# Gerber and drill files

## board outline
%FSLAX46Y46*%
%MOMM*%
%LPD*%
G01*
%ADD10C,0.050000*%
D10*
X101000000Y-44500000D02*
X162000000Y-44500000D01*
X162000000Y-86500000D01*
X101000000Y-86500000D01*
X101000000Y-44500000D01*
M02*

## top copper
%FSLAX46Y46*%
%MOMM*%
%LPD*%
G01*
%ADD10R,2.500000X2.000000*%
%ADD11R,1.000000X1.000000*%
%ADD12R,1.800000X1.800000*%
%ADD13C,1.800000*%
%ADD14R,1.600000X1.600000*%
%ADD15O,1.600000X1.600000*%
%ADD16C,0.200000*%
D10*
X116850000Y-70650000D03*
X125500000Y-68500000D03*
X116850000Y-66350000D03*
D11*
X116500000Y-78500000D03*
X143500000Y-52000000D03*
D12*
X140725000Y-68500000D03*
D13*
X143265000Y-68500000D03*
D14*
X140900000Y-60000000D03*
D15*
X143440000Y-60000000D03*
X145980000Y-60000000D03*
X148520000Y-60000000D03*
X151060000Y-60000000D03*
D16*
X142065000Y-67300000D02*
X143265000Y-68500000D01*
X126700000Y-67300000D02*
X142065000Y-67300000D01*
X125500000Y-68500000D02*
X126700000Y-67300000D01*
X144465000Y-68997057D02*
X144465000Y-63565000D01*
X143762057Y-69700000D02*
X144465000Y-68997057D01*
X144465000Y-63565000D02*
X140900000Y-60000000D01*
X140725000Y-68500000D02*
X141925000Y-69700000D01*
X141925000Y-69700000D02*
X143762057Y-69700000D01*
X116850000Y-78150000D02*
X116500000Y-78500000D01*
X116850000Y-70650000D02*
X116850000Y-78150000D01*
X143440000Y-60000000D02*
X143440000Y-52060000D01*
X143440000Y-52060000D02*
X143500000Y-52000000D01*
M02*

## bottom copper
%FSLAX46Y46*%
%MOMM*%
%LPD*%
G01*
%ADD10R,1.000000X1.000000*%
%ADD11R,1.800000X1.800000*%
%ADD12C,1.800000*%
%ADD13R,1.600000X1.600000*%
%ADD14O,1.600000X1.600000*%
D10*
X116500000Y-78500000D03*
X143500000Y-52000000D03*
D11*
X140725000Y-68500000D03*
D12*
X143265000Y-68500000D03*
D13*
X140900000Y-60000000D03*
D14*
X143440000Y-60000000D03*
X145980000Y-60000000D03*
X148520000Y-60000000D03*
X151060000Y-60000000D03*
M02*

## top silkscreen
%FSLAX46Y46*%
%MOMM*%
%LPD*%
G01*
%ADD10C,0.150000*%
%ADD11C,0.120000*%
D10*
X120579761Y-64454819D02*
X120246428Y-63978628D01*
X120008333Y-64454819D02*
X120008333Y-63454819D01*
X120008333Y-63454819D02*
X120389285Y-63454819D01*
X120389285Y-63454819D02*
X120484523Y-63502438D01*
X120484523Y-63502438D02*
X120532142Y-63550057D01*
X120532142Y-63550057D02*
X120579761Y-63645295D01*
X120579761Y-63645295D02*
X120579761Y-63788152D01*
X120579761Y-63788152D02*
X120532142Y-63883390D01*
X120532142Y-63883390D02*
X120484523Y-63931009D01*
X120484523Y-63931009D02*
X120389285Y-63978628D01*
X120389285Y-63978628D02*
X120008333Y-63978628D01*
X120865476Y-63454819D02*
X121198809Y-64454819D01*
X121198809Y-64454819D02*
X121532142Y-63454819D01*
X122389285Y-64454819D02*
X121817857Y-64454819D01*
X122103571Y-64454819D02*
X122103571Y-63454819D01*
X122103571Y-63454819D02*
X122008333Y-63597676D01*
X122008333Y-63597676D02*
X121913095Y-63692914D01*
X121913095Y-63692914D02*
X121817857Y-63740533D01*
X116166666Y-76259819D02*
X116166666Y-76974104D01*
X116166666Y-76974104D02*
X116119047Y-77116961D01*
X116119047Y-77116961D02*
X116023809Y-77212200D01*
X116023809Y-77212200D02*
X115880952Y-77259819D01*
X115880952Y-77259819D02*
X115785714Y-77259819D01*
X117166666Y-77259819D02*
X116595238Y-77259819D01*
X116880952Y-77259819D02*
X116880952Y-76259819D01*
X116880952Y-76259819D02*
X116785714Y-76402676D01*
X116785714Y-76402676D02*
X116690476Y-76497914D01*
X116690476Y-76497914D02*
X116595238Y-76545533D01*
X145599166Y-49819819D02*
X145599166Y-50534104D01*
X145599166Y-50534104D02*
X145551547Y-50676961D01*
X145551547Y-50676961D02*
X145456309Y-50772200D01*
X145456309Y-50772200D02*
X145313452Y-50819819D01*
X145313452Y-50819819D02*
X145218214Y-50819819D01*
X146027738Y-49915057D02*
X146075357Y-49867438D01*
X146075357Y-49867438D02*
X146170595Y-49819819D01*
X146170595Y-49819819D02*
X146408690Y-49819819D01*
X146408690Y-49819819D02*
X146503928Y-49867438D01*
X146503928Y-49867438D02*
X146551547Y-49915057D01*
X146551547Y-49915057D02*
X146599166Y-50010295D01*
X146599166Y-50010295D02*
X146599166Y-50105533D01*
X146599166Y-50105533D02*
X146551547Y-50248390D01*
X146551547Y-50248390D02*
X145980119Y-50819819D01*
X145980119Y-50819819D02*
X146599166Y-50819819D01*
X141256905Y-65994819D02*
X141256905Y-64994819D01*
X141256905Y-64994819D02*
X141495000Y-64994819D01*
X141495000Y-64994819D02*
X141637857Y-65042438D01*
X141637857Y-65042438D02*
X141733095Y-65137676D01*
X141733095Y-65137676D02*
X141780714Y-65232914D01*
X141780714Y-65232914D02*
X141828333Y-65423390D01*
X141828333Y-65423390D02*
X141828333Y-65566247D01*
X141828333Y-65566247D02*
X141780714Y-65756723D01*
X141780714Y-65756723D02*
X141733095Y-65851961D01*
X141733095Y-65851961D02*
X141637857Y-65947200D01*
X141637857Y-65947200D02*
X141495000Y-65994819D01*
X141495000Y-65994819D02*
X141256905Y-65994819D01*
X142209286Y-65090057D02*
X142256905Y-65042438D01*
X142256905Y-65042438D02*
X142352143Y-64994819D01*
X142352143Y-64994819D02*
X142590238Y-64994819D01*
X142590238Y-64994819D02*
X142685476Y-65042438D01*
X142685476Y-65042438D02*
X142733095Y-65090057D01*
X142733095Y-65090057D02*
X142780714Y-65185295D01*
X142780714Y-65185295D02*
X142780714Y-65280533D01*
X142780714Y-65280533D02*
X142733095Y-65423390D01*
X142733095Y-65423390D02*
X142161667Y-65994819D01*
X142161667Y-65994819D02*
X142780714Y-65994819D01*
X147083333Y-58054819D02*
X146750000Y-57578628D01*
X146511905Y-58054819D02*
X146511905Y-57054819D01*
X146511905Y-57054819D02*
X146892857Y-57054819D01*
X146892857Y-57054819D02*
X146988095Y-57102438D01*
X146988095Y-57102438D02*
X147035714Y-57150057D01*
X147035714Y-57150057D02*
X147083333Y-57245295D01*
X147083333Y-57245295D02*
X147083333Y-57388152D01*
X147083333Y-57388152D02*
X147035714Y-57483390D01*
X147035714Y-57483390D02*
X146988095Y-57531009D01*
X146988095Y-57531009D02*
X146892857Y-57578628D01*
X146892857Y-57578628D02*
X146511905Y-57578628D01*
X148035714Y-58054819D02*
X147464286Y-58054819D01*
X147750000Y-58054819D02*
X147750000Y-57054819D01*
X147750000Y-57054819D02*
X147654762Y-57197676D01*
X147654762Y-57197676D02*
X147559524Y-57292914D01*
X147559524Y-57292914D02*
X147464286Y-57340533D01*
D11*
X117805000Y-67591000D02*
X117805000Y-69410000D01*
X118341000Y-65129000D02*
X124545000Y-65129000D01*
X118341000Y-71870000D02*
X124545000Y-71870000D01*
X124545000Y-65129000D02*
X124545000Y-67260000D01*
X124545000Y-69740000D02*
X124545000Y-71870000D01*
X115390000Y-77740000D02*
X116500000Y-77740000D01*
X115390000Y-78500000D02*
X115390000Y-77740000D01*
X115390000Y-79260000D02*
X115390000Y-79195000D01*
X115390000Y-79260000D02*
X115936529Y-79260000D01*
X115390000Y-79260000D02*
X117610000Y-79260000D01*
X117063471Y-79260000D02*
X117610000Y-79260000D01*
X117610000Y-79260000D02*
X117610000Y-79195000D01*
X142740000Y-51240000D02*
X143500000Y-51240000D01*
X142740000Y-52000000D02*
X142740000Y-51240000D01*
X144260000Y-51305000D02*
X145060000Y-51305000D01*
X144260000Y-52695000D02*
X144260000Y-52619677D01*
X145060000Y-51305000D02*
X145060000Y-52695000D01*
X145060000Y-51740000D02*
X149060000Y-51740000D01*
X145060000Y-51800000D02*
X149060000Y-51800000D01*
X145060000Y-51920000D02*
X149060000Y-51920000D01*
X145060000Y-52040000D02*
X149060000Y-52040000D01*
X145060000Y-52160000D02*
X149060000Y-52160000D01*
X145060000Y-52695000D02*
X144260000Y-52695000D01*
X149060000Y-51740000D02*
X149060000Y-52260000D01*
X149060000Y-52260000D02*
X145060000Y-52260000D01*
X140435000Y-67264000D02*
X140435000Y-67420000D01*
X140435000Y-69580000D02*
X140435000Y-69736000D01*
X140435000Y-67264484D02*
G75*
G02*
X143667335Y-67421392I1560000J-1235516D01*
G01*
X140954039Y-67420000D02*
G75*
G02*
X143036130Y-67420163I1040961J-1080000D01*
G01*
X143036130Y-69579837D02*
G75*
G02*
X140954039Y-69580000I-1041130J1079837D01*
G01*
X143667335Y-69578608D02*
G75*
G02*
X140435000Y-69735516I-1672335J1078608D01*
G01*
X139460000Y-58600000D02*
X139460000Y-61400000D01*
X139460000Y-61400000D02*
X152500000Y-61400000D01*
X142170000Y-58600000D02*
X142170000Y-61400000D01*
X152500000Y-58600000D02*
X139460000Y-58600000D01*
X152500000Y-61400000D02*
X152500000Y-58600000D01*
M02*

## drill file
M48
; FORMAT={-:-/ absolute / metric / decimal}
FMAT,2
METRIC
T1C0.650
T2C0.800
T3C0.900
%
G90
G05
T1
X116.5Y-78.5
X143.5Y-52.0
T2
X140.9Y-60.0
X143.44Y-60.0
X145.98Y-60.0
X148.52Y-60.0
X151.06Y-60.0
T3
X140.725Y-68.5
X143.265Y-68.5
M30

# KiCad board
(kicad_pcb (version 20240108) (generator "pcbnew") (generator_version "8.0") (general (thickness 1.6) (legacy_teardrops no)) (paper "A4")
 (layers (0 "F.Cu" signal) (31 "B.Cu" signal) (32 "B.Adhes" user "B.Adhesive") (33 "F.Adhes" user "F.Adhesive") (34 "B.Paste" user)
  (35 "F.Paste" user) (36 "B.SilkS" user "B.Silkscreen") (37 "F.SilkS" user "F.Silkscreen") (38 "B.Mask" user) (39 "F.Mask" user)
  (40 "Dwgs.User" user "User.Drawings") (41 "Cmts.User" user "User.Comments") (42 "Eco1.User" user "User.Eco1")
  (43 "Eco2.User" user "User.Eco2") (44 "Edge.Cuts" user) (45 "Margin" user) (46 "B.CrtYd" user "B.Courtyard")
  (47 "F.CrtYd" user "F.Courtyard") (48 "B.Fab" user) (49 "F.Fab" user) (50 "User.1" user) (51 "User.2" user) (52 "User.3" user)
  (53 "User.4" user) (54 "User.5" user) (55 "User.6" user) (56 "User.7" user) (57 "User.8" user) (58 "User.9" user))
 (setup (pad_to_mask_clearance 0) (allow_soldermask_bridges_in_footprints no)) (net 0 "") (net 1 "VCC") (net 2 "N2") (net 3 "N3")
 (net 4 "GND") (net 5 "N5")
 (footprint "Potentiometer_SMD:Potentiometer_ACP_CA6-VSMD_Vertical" (layer "F.Cu") (at 121.175 68.5)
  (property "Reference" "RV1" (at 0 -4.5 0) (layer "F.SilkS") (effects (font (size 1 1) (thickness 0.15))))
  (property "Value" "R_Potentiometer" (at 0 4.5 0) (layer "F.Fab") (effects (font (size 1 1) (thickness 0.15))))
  (fp_line (start -3.37 -0.909) (end -3.37 0.91) (stroke (width 0.12) (type solid)) (layer "F.SilkS"))
  (fp_line (start -2.834 -3.371) (end 3.37 -3.371) (stroke (width 0.12) (type solid)) (layer "F.SilkS"))
  (fp_line (start -2.834 3.37) (end 3.37 3.37) (stroke (width 0.12) (type solid)) (layer "F.SilkS"))
  (fp_line (start 3.37 -3.371) (end 3.37 -1.24) (stroke (width 0.12) (type solid)) (layer "F.SilkS"))
  (fp_line (start 3.37 1.24) (end 3.37 3.37) (stroke (width 0.12) (type solid)) (layer "F.SilkS"))
  (pad "1" smd rect (at -4.325 2.15) (size 2.5 2) (layers "F.Cu" "F.Paste" "F.Mask") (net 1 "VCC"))
  (pad "2" smd rect (at 4.325 0) (size 2.5 2) (layers "F.Cu" "F.Paste" "F.Mask") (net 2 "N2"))
  (pad "3" smd rect (at -4.325 -2.15) (size 2.5 2) (layers "F.Cu" "F.Paste" "F.Mask") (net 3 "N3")))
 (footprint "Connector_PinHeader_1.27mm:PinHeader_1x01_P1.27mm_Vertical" (layer "F.Cu") (at 116.5 78.5)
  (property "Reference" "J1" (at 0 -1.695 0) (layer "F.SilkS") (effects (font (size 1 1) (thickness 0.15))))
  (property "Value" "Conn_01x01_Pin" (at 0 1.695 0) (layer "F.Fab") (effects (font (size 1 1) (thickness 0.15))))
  (fp_line (start -1.11 -0.76) (end 0 -0.76) (stroke (width 0.12) (type solid)) (layer "F.SilkS"))
  (fp_line (start -1.11 0) (end -1.11 -0.76) (stroke (width 0.12) (type solid)) (layer "F.SilkS"))
  (fp_line (start -1.11 0.76) (end -1.11 0.695) (stroke (width 0.12) (type solid)) (layer "F.SilkS"))
  (fp_line (start -1.11 0.76) (end -0.563471 0.76) (stroke (width 0.12) (type solid)) (layer "F.SilkS"))
  (fp_line (start -1.11 0.76) (end 1.11 0.76) (stroke (width 0.12) (type solid)) (layer "F.SilkS"))
  (fp_line (start 0.563471 0.76) (end 1.11 0.76) (stroke (width 0.12) (type solid)) (layer "F.SilkS"))
  (fp_line (start 1.11 0.76) (end 1.11 0.695) (stroke (width 0.12) (type solid)) (layer "F.SilkS"))
  (pad "1" thru_hole rect (at 0 0) (size 1 1) (drill 0.65) (layers "*.Cu" "*.Mask") (remove_unused_layers no) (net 1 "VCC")))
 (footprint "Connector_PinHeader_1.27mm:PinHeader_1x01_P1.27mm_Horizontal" (layer "F.Cu") (at 143.5 52)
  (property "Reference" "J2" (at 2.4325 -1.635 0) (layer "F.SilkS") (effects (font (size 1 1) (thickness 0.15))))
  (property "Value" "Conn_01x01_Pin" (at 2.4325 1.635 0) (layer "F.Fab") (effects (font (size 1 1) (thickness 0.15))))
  (fp_line (start -0.76 -0.76) (end 0 -0.76) (stroke (width 0.12) (type solid)) (layer "F.SilkS"))
  (fp_line (start -0.76 0) (end -0.76 -0.76) (stroke (width 0.12) (type solid)) (layer "F.SilkS"))
  (fp_line (start 0.76 -0.695) (end 1.56 -0.695) (stroke (width 0.12) (type solid)) (layer "F.SilkS"))
  (fp_line (start 0.76 0.695) (end 0.76 0.619677) (stroke (width 0.12) (type solid)) (layer "F.SilkS"))
  (fp_line (start 1.56 -0.695) (end 1.56 0.695) (stroke (width 0.12) (type solid)) (layer "F.SilkS"))
  (fp_line (start 1.56 -0.26) (end 5.56 -0.26) (stroke (width 0.12) (type solid)) (layer "F.SilkS"))
  (fp_line (start 1.56 -0.2) (end 5.56 -0.2) (stroke (width 0.12) (type solid)) (layer "F.SilkS"))
  (fp_line (start 1.56 -0.08) (end 5.56 -0.08) (stroke (width 0.12) (type solid)) (layer "F.SilkS"))
  (fp_line (start 1.56 0.04) (end 5.56 0.04) (stroke (width 0.12) (type solid)) (layer "F.SilkS"))
  (fp_line (start 1.56 0.16) (end 5.56 0.16) (stroke (width 0.12) (type solid)) (layer "F.SilkS"))
  (fp_line (start 1.56 0.695) (end 0.76 0.695) (stroke (width 0.12) (type solid)) (layer "F.SilkS"))
  (fp_line (start 5.56 -0.26) (end 5.56 0.26) (stroke (width 0.12) (type solid)) (layer "F.SilkS"))
  (fp_line (start 5.56 0.26) (end 1.56 0.26) (stroke (width 0.12) (type solid)) (layer "F.SilkS"))
  (pad "1" thru_hole rect (at 0 0) (size 1 1) (drill 0.65) (layers "*.Cu" "*.Mask") (remove_unused_layers no) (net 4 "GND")))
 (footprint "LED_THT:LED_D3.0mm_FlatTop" (layer "F.Cu") (at 140.725 68.5)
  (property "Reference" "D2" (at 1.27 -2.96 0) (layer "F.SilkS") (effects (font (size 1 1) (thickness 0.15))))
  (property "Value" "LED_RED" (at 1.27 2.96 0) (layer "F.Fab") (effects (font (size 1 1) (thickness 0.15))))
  (fp_line (start -0.29 -1.236) (end -0.29 -1.08) (stroke (width 0.12) (type solid)) (layer "F.SilkS"))
  (fp_line (start -0.29 1.08) (end -0.29 1.236) (stroke (width 0.12) (type solid)) (layer "F.SilkS"))
  (fp_arc (start -0.29 -1.235516) (mid 1.366487 -1.987659) (end 2.942335 -1.078608) (stroke (width 0.12) (type solid)) (layer "F.SilkS"))
  (fp_arc (start 0.229039 -1.08) (mid 1.270117 -1.5) (end 2.31113 -1.079837) (stroke (width 0.12) (type solid)) (layer "F.SilkS"))
  (fp_arc (start 2.31113 1.079837) (mid 1.270117 1.5) (end 0.229039 1.08) (stroke (width 0.12) (type solid)) (layer "F.SilkS"))
  (fp_arc (start 2.942335 1.078608) (mid 1.366487 1.987659) (end -0.29 1.235516) (stroke (width 0.12) (type solid)) (layer "F.SilkS"))
  (pad "1" thru_hole rect (at 0 0) (size 1.8 1.8) (drill 0.9) (layers "*.Cu" "*.Mask") (remove_unused_layers no) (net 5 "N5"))
  (pad "2" thru_hole circle (at 2.54 0) (size 1.8 1.8) (drill 0.9) (layers "*.Cu" "*.Mask") (remove_unused_layers no) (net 2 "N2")))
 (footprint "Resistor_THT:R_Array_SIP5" (layer "F.Cu") (at 140.9 60)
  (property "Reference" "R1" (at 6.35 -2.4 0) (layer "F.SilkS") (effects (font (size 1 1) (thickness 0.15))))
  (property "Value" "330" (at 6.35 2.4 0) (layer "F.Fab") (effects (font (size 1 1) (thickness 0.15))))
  (fp_line (start -1.44 -1.4) (end -1.44 1.4) (stroke (width 0.12) (type solid)) (layer "F.SilkS"))
  (fp_line (start -1.44 1.4) (end 11.6 1.4) (stroke (width 0.12) (type solid)) (layer "F.SilkS"))
  (fp_line (start 1.27 -1.4) (end 1.27 1.4) (stroke (width 0.12) (type solid)) (layer "F.SilkS"))
  (fp_line (start 11.6 -1.4) (end -1.44 -1.4) (stroke (width 0.12) (type solid)) (layer "F.SilkS"))
  (fp_line (start 11.6 1.4) (end 11.6 -1.4) (stroke (width 0.12) (type solid)) (layer "F.SilkS"))
  (pad "1" thru_hole rect (at 0 0) (size 1.6 1.6) (drill 0.8) (layers "*.Cu" "*.Mask") (remove_unused_layers no) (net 5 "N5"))
  (pad "2" thru_hole oval (at 2.54 0) (size 1.6 1.6) (drill 0.8) (layers "*.Cu" "*.Mask") (remove_unused_layers no) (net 4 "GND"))
  (pad "3" thru_hole oval (at 5.08 0) (size 1.6 1.6) (drill 0.8) (layers "*.Cu" "*.Mask") (remove_unused_layers no))
  (pad "4" thru_hole oval (at 7.62 0) (size 1.6 1.6) (drill 0.8) (layers "*.Cu" "*.Mask") (remove_unused_layers no))
  (pad "5" thru_hole oval (at 10.16 0) (size 1.6 1.6) (drill 0.8) (layers "*.Cu" "*.Mask") (remove_unused_layers no)))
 (gr_rect (start 101 44.5) (end 162 86.5) (stroke (width 0.05) (type default)) (fill none) (layer "Edge.Cuts"))
 (segment (start 142.065 67.3) (end 143.265 68.5) (width 0.2) (layer "F.Cu") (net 2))
 (segment (start 126.7 67.3) (end 142.065 67.3) (width 0.2) (layer "F.Cu") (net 2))
 (segment (start 125.5 68.5) (end 126.7 67.3) (width 0.2) (layer "F.Cu") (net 2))
 (segment (start 144.465 68.997057) (end 144.465 63.565) (width 0.2) (layer "F.Cu") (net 5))
 (segment (start 143.762057 69.7) (end 144.465 68.997057) (width 0.2) (layer "F.Cu") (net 5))
 (segment (start 144.465 63.565) (end 140.9 60) (width 0.2) (layer "F.Cu") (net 5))
 (segment (start 140.725 68.5) (end 141.925 69.7) (width 0.2) (layer "F.Cu") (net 5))
 (segment (start 141.925 69.7) (end 143.762057 69.7) (width 0.2) (layer "F.Cu") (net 5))
 (segment (start 116.85 78.15) (end 116.5 78.5) (width 0.2) (layer "F.Cu") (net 1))
 (segment (start 116.85 70.65) (end 116.85 78.15) (width 0.2) (layer "F.Cu") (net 1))
 (segment (start 143.44 60) (end 143.44 52.06) (width 0.2) (layer "F.Cu") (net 4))
 (segment (start 143.44 52.06) (end 143.5 52) (width 0.2) (layer "F.Cu") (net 4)))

